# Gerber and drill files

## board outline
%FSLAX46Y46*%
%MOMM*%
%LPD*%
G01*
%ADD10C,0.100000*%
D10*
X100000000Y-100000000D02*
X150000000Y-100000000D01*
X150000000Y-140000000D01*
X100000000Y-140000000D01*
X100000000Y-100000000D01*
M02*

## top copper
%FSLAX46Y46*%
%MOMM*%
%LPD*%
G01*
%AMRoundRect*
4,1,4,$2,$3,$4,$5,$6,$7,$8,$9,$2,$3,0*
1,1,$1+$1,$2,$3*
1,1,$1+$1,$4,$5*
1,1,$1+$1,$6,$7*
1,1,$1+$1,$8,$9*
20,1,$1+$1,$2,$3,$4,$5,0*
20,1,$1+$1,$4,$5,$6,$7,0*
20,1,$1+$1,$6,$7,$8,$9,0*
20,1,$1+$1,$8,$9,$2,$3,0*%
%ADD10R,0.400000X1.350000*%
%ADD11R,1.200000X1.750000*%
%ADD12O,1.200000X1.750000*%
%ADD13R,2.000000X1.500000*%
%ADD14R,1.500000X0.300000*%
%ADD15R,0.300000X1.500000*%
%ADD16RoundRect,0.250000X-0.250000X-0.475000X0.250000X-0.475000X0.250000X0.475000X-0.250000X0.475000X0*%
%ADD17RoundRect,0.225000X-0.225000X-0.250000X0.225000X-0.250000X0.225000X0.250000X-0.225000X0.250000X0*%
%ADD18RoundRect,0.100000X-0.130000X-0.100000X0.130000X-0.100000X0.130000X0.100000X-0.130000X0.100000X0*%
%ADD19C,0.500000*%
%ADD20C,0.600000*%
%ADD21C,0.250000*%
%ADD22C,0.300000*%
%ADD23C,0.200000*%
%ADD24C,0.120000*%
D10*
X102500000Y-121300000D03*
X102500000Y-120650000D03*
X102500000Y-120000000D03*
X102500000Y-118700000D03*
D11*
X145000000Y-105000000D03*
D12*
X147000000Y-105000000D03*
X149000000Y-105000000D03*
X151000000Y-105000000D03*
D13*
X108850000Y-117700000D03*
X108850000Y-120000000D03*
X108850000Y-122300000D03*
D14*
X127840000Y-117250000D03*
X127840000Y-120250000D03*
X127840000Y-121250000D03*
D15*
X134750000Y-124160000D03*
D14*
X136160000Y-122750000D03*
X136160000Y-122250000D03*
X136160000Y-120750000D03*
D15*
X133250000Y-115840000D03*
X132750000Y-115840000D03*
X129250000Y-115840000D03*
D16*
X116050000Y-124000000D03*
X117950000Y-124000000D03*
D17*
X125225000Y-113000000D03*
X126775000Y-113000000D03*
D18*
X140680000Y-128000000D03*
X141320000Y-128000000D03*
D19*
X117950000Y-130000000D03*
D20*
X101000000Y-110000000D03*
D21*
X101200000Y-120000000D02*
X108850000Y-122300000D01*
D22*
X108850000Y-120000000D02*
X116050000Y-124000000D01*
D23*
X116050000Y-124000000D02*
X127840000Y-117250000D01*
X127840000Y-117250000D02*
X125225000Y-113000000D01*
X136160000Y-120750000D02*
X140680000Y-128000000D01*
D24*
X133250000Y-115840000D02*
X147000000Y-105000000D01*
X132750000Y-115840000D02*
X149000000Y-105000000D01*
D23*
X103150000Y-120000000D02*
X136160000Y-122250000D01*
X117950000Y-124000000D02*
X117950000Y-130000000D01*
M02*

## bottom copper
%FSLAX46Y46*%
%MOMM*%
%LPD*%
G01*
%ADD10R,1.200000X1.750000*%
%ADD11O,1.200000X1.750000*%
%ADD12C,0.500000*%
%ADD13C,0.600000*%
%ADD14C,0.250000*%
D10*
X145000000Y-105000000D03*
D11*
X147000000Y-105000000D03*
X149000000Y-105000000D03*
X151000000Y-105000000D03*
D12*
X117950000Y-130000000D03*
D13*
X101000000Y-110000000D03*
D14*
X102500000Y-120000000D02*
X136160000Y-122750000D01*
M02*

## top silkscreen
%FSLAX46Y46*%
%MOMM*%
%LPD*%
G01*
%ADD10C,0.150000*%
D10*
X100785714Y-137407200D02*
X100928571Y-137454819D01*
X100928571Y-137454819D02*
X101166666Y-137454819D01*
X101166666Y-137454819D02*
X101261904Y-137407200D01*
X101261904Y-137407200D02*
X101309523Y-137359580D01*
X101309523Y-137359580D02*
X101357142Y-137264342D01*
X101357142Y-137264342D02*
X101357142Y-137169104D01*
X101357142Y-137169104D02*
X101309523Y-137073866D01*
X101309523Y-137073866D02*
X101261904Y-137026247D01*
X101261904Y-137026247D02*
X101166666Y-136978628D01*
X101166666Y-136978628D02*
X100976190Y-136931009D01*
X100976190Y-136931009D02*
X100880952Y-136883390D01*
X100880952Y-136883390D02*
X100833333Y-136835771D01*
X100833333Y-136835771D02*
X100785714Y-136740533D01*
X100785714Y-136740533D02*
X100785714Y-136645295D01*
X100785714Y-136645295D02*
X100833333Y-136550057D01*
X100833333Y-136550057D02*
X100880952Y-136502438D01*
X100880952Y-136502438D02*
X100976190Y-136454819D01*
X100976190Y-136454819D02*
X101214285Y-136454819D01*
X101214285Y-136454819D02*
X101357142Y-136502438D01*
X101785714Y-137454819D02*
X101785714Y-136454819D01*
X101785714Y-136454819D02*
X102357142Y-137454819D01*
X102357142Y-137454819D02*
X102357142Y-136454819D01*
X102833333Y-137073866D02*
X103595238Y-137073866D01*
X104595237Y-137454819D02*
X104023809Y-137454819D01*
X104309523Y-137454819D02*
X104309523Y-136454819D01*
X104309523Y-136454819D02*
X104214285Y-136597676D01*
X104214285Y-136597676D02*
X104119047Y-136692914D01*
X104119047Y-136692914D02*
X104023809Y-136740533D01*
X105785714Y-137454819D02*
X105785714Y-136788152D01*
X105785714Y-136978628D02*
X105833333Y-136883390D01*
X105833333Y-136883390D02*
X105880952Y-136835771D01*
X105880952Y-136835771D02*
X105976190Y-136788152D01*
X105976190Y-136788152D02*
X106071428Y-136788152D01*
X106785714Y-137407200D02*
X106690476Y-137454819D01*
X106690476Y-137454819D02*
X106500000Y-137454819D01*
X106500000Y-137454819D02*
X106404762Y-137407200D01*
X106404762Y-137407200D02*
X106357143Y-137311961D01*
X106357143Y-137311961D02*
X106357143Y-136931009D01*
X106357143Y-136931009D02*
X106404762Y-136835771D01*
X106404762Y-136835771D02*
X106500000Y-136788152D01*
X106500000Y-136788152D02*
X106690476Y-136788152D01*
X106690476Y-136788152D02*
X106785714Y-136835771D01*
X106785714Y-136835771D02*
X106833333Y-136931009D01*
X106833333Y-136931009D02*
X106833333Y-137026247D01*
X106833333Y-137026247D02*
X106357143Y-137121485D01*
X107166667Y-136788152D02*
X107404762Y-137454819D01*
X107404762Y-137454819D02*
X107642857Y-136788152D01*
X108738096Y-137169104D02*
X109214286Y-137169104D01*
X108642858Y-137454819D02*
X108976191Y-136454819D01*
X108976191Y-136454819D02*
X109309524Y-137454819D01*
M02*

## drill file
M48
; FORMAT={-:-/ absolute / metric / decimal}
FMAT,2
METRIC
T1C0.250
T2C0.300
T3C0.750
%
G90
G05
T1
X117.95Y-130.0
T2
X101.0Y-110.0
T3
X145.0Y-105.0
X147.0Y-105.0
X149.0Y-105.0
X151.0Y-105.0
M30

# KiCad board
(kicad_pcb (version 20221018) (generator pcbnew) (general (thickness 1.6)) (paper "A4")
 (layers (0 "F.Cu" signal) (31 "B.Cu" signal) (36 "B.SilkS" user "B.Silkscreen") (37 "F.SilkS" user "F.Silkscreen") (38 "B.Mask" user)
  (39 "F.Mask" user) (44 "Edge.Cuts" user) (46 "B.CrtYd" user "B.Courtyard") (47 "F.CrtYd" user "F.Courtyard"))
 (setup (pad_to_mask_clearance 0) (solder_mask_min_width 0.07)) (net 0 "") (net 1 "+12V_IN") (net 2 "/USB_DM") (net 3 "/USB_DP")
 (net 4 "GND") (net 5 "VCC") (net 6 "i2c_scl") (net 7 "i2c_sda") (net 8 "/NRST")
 (gr_rect (start 100 100) (end 150 140) (layer "Edge.Cuts") (width 0.1))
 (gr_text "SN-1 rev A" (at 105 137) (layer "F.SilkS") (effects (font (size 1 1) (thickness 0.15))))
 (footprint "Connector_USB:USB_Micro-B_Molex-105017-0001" (layer "F.Cu") (at 102.5 120 90) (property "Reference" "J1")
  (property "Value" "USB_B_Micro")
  (pad "1" smd rect (at -1.3 0) (size 0.4 1.35) (layers "F.Cu" "F.Mask") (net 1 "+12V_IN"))
  (pad "2" smd rect (at -0.65 0) (size 0.4 1.35) (layers "F.Cu" "F.Mask") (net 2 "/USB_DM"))
  (pad "3" smd rect (at 0 0) (size 0.4 1.35) (layers "F.Cu" "F.Mask") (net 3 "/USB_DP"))
  (pad "5" smd rect (at 1.3 0) (size 0.4 1.35) (layers "F.Cu" "F.Mask") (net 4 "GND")))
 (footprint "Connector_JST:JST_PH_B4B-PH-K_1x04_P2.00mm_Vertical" (layer "F.Cu") (at 145 105 0) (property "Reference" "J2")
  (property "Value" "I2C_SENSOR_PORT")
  (pad "1" thru_hole rect (at 0 0) (size 1.2 1.75) (drill 0.75) (layers "*.Cu" "*.Mask") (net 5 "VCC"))
  (pad "2" thru_hole oval (at 2 0) (size 1.2 1.75) (drill 0.75) (layers "*.Cu" "*.Mask") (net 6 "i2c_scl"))
  (pad "3" thru_hole oval (at 4 0) (size 1.2 1.75) (drill 0.75) (layers "*.Cu" "*.Mask") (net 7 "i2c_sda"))
  (pad "4" thru_hole oval (at 6 0) (size 1.2 1.75) (drill 0.75) (layers "*.Cu" "*.Mask") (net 4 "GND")))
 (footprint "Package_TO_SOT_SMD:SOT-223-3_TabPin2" (layer "F.Cu") (at 112 120 0) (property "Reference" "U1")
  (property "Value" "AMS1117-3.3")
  (pad "1" smd rect (at -3.15 -2.3) (size 2 1.5) (layers "F.Cu" "F.Mask") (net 4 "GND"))
  (pad "2" smd rect (at -3.15 0) (size 2 1.5) (layers "F.Cu" "F.Mask") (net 5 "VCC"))
  (pad "3" smd rect (at -3.15 2.3) (size 2 1.5) (layers "F.Cu" "F.Mask") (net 1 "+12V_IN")))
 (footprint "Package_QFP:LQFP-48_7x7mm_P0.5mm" (layer "F.Cu") (at 132 120 0) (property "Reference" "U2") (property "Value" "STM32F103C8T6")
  (pad "1" smd rect (at -4.16 -2.75) (size 1.5 0.3) (layers "F.Cu" "F.Mask") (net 5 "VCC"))
  (pad "7" smd rect (at -4.16 0.25) (size 1.5 0.3) (layers "F.Cu" "F.Mask") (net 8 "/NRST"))
  (pad "9" smd rect (at -4.16 1.25) (size 1.5 0.3) (layers "F.Cu" "F.Mask") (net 5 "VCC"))
  (pad "24" smd rect (at 2.75 4.16) (size 0.3 1.5) (layers "F.Cu" "F.Mask") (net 5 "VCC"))
  (pad "32" smd rect (at 4.16 2.75) (size 1.5 0.3) (layers "F.Cu" "F.Mask") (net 2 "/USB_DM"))
  (pad "33" smd rect (at 4.16 2.25) (size 1.5 0.3) (layers "F.Cu" "F.Mask") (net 3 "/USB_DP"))
  (pad "36" smd rect (at 4.16 0.75) (size 1.5 0.3) (layers "F.Cu" "F.Mask") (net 5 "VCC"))
  (pad "42" smd rect (at 1.25 -4.16) (size 0.3 1.5) (layers "F.Cu" "F.Mask") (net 6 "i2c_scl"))
  (pad "43" smd rect (at 0.75 -4.16) (size 0.3 1.5) (layers "F.Cu" "F.Mask") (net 7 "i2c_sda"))
  (pad "48" smd rect (at -2.75 -4.16) (size 0.3 1.5) (layers "F.Cu" "F.Mask") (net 5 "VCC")))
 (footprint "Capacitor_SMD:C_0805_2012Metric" (layer "F.Cu") (at 117 124 0) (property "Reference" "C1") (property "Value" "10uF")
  (pad "1" smd roundrect (at -0.95 0) (size 1 1.45) (layers "F.Cu" "F.Mask") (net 5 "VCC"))
  (pad "2" smd roundrect (at 0.95 0) (size 1 1.45) (layers "F.Cu" "F.Mask") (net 4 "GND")))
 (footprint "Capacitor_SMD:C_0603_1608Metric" (layer "F.Cu") (at 126 113 0) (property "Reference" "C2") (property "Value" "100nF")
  (pad "1" smd roundrect (at -0.775 0) (size 0.9 0.95) (layers "F.Cu" "F.Mask") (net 5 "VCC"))
  (pad "2" smd roundrect (at 0.775 0) (size 0.9 0.95) (layers "F.Cu" "F.Mask") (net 4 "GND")))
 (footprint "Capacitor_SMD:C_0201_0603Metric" (layer "F.Cu") (at 141 128 0) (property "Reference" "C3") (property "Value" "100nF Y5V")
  (pad "1" smd roundrect (at -0.32 0) (size 0.46 0.4) (layers "F.Cu" "F.Mask") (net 5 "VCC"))
  (pad "2" smd roundrect (at 0.32 0) (size 0.46 0.4) (layers "F.Cu" "F.Mask") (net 4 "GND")))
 (segment (start 101.2 120) (end 108.85 122.3) (width 0.25) (layer "F.Cu") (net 1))
 (segment (start 108.85 120) (end 116.05 124) (width 0.3) (layer "F.Cu") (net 5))
 (segment (start 116.05 124) (end 127.84 117.25) (width 0.2) (layer "F.Cu") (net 5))
 (segment (start 127.84 117.25) (end 125.225 113) (width 0.2) (layer "F.Cu") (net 5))
 (segment (start 136.16 120.75) (end 140.68 128) (width 0.2) (layer "F.Cu") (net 5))
 (segment (start 133.25 115.84) (end 147 105) (width 0.12) (layer "F.Cu") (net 6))
 (segment (start 132.75 115.84) (end 149 105) (width 0.12) (layer "F.Cu") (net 7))
 (segment (start 103.15 120) (end 136.16 122.25) (width 0.2) (layer "F.Cu") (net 3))
 (segment (start 102.5 120) (end 136.16 122.75) (width 0.25) (layer "B.Cu") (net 2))
 (segment (start 117.95 124) (end 117.95 130) (width 0.2) (layer "F.Cu") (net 4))
 (via (at 117.95 130) (size 0.5) (drill 0.25) (layers "F.Cu" "B.Cu") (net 4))
 (via (at 101.0 110.0) (size 0.6) (drill 0.3) (layers "F.Cu" "B.Cu") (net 4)))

